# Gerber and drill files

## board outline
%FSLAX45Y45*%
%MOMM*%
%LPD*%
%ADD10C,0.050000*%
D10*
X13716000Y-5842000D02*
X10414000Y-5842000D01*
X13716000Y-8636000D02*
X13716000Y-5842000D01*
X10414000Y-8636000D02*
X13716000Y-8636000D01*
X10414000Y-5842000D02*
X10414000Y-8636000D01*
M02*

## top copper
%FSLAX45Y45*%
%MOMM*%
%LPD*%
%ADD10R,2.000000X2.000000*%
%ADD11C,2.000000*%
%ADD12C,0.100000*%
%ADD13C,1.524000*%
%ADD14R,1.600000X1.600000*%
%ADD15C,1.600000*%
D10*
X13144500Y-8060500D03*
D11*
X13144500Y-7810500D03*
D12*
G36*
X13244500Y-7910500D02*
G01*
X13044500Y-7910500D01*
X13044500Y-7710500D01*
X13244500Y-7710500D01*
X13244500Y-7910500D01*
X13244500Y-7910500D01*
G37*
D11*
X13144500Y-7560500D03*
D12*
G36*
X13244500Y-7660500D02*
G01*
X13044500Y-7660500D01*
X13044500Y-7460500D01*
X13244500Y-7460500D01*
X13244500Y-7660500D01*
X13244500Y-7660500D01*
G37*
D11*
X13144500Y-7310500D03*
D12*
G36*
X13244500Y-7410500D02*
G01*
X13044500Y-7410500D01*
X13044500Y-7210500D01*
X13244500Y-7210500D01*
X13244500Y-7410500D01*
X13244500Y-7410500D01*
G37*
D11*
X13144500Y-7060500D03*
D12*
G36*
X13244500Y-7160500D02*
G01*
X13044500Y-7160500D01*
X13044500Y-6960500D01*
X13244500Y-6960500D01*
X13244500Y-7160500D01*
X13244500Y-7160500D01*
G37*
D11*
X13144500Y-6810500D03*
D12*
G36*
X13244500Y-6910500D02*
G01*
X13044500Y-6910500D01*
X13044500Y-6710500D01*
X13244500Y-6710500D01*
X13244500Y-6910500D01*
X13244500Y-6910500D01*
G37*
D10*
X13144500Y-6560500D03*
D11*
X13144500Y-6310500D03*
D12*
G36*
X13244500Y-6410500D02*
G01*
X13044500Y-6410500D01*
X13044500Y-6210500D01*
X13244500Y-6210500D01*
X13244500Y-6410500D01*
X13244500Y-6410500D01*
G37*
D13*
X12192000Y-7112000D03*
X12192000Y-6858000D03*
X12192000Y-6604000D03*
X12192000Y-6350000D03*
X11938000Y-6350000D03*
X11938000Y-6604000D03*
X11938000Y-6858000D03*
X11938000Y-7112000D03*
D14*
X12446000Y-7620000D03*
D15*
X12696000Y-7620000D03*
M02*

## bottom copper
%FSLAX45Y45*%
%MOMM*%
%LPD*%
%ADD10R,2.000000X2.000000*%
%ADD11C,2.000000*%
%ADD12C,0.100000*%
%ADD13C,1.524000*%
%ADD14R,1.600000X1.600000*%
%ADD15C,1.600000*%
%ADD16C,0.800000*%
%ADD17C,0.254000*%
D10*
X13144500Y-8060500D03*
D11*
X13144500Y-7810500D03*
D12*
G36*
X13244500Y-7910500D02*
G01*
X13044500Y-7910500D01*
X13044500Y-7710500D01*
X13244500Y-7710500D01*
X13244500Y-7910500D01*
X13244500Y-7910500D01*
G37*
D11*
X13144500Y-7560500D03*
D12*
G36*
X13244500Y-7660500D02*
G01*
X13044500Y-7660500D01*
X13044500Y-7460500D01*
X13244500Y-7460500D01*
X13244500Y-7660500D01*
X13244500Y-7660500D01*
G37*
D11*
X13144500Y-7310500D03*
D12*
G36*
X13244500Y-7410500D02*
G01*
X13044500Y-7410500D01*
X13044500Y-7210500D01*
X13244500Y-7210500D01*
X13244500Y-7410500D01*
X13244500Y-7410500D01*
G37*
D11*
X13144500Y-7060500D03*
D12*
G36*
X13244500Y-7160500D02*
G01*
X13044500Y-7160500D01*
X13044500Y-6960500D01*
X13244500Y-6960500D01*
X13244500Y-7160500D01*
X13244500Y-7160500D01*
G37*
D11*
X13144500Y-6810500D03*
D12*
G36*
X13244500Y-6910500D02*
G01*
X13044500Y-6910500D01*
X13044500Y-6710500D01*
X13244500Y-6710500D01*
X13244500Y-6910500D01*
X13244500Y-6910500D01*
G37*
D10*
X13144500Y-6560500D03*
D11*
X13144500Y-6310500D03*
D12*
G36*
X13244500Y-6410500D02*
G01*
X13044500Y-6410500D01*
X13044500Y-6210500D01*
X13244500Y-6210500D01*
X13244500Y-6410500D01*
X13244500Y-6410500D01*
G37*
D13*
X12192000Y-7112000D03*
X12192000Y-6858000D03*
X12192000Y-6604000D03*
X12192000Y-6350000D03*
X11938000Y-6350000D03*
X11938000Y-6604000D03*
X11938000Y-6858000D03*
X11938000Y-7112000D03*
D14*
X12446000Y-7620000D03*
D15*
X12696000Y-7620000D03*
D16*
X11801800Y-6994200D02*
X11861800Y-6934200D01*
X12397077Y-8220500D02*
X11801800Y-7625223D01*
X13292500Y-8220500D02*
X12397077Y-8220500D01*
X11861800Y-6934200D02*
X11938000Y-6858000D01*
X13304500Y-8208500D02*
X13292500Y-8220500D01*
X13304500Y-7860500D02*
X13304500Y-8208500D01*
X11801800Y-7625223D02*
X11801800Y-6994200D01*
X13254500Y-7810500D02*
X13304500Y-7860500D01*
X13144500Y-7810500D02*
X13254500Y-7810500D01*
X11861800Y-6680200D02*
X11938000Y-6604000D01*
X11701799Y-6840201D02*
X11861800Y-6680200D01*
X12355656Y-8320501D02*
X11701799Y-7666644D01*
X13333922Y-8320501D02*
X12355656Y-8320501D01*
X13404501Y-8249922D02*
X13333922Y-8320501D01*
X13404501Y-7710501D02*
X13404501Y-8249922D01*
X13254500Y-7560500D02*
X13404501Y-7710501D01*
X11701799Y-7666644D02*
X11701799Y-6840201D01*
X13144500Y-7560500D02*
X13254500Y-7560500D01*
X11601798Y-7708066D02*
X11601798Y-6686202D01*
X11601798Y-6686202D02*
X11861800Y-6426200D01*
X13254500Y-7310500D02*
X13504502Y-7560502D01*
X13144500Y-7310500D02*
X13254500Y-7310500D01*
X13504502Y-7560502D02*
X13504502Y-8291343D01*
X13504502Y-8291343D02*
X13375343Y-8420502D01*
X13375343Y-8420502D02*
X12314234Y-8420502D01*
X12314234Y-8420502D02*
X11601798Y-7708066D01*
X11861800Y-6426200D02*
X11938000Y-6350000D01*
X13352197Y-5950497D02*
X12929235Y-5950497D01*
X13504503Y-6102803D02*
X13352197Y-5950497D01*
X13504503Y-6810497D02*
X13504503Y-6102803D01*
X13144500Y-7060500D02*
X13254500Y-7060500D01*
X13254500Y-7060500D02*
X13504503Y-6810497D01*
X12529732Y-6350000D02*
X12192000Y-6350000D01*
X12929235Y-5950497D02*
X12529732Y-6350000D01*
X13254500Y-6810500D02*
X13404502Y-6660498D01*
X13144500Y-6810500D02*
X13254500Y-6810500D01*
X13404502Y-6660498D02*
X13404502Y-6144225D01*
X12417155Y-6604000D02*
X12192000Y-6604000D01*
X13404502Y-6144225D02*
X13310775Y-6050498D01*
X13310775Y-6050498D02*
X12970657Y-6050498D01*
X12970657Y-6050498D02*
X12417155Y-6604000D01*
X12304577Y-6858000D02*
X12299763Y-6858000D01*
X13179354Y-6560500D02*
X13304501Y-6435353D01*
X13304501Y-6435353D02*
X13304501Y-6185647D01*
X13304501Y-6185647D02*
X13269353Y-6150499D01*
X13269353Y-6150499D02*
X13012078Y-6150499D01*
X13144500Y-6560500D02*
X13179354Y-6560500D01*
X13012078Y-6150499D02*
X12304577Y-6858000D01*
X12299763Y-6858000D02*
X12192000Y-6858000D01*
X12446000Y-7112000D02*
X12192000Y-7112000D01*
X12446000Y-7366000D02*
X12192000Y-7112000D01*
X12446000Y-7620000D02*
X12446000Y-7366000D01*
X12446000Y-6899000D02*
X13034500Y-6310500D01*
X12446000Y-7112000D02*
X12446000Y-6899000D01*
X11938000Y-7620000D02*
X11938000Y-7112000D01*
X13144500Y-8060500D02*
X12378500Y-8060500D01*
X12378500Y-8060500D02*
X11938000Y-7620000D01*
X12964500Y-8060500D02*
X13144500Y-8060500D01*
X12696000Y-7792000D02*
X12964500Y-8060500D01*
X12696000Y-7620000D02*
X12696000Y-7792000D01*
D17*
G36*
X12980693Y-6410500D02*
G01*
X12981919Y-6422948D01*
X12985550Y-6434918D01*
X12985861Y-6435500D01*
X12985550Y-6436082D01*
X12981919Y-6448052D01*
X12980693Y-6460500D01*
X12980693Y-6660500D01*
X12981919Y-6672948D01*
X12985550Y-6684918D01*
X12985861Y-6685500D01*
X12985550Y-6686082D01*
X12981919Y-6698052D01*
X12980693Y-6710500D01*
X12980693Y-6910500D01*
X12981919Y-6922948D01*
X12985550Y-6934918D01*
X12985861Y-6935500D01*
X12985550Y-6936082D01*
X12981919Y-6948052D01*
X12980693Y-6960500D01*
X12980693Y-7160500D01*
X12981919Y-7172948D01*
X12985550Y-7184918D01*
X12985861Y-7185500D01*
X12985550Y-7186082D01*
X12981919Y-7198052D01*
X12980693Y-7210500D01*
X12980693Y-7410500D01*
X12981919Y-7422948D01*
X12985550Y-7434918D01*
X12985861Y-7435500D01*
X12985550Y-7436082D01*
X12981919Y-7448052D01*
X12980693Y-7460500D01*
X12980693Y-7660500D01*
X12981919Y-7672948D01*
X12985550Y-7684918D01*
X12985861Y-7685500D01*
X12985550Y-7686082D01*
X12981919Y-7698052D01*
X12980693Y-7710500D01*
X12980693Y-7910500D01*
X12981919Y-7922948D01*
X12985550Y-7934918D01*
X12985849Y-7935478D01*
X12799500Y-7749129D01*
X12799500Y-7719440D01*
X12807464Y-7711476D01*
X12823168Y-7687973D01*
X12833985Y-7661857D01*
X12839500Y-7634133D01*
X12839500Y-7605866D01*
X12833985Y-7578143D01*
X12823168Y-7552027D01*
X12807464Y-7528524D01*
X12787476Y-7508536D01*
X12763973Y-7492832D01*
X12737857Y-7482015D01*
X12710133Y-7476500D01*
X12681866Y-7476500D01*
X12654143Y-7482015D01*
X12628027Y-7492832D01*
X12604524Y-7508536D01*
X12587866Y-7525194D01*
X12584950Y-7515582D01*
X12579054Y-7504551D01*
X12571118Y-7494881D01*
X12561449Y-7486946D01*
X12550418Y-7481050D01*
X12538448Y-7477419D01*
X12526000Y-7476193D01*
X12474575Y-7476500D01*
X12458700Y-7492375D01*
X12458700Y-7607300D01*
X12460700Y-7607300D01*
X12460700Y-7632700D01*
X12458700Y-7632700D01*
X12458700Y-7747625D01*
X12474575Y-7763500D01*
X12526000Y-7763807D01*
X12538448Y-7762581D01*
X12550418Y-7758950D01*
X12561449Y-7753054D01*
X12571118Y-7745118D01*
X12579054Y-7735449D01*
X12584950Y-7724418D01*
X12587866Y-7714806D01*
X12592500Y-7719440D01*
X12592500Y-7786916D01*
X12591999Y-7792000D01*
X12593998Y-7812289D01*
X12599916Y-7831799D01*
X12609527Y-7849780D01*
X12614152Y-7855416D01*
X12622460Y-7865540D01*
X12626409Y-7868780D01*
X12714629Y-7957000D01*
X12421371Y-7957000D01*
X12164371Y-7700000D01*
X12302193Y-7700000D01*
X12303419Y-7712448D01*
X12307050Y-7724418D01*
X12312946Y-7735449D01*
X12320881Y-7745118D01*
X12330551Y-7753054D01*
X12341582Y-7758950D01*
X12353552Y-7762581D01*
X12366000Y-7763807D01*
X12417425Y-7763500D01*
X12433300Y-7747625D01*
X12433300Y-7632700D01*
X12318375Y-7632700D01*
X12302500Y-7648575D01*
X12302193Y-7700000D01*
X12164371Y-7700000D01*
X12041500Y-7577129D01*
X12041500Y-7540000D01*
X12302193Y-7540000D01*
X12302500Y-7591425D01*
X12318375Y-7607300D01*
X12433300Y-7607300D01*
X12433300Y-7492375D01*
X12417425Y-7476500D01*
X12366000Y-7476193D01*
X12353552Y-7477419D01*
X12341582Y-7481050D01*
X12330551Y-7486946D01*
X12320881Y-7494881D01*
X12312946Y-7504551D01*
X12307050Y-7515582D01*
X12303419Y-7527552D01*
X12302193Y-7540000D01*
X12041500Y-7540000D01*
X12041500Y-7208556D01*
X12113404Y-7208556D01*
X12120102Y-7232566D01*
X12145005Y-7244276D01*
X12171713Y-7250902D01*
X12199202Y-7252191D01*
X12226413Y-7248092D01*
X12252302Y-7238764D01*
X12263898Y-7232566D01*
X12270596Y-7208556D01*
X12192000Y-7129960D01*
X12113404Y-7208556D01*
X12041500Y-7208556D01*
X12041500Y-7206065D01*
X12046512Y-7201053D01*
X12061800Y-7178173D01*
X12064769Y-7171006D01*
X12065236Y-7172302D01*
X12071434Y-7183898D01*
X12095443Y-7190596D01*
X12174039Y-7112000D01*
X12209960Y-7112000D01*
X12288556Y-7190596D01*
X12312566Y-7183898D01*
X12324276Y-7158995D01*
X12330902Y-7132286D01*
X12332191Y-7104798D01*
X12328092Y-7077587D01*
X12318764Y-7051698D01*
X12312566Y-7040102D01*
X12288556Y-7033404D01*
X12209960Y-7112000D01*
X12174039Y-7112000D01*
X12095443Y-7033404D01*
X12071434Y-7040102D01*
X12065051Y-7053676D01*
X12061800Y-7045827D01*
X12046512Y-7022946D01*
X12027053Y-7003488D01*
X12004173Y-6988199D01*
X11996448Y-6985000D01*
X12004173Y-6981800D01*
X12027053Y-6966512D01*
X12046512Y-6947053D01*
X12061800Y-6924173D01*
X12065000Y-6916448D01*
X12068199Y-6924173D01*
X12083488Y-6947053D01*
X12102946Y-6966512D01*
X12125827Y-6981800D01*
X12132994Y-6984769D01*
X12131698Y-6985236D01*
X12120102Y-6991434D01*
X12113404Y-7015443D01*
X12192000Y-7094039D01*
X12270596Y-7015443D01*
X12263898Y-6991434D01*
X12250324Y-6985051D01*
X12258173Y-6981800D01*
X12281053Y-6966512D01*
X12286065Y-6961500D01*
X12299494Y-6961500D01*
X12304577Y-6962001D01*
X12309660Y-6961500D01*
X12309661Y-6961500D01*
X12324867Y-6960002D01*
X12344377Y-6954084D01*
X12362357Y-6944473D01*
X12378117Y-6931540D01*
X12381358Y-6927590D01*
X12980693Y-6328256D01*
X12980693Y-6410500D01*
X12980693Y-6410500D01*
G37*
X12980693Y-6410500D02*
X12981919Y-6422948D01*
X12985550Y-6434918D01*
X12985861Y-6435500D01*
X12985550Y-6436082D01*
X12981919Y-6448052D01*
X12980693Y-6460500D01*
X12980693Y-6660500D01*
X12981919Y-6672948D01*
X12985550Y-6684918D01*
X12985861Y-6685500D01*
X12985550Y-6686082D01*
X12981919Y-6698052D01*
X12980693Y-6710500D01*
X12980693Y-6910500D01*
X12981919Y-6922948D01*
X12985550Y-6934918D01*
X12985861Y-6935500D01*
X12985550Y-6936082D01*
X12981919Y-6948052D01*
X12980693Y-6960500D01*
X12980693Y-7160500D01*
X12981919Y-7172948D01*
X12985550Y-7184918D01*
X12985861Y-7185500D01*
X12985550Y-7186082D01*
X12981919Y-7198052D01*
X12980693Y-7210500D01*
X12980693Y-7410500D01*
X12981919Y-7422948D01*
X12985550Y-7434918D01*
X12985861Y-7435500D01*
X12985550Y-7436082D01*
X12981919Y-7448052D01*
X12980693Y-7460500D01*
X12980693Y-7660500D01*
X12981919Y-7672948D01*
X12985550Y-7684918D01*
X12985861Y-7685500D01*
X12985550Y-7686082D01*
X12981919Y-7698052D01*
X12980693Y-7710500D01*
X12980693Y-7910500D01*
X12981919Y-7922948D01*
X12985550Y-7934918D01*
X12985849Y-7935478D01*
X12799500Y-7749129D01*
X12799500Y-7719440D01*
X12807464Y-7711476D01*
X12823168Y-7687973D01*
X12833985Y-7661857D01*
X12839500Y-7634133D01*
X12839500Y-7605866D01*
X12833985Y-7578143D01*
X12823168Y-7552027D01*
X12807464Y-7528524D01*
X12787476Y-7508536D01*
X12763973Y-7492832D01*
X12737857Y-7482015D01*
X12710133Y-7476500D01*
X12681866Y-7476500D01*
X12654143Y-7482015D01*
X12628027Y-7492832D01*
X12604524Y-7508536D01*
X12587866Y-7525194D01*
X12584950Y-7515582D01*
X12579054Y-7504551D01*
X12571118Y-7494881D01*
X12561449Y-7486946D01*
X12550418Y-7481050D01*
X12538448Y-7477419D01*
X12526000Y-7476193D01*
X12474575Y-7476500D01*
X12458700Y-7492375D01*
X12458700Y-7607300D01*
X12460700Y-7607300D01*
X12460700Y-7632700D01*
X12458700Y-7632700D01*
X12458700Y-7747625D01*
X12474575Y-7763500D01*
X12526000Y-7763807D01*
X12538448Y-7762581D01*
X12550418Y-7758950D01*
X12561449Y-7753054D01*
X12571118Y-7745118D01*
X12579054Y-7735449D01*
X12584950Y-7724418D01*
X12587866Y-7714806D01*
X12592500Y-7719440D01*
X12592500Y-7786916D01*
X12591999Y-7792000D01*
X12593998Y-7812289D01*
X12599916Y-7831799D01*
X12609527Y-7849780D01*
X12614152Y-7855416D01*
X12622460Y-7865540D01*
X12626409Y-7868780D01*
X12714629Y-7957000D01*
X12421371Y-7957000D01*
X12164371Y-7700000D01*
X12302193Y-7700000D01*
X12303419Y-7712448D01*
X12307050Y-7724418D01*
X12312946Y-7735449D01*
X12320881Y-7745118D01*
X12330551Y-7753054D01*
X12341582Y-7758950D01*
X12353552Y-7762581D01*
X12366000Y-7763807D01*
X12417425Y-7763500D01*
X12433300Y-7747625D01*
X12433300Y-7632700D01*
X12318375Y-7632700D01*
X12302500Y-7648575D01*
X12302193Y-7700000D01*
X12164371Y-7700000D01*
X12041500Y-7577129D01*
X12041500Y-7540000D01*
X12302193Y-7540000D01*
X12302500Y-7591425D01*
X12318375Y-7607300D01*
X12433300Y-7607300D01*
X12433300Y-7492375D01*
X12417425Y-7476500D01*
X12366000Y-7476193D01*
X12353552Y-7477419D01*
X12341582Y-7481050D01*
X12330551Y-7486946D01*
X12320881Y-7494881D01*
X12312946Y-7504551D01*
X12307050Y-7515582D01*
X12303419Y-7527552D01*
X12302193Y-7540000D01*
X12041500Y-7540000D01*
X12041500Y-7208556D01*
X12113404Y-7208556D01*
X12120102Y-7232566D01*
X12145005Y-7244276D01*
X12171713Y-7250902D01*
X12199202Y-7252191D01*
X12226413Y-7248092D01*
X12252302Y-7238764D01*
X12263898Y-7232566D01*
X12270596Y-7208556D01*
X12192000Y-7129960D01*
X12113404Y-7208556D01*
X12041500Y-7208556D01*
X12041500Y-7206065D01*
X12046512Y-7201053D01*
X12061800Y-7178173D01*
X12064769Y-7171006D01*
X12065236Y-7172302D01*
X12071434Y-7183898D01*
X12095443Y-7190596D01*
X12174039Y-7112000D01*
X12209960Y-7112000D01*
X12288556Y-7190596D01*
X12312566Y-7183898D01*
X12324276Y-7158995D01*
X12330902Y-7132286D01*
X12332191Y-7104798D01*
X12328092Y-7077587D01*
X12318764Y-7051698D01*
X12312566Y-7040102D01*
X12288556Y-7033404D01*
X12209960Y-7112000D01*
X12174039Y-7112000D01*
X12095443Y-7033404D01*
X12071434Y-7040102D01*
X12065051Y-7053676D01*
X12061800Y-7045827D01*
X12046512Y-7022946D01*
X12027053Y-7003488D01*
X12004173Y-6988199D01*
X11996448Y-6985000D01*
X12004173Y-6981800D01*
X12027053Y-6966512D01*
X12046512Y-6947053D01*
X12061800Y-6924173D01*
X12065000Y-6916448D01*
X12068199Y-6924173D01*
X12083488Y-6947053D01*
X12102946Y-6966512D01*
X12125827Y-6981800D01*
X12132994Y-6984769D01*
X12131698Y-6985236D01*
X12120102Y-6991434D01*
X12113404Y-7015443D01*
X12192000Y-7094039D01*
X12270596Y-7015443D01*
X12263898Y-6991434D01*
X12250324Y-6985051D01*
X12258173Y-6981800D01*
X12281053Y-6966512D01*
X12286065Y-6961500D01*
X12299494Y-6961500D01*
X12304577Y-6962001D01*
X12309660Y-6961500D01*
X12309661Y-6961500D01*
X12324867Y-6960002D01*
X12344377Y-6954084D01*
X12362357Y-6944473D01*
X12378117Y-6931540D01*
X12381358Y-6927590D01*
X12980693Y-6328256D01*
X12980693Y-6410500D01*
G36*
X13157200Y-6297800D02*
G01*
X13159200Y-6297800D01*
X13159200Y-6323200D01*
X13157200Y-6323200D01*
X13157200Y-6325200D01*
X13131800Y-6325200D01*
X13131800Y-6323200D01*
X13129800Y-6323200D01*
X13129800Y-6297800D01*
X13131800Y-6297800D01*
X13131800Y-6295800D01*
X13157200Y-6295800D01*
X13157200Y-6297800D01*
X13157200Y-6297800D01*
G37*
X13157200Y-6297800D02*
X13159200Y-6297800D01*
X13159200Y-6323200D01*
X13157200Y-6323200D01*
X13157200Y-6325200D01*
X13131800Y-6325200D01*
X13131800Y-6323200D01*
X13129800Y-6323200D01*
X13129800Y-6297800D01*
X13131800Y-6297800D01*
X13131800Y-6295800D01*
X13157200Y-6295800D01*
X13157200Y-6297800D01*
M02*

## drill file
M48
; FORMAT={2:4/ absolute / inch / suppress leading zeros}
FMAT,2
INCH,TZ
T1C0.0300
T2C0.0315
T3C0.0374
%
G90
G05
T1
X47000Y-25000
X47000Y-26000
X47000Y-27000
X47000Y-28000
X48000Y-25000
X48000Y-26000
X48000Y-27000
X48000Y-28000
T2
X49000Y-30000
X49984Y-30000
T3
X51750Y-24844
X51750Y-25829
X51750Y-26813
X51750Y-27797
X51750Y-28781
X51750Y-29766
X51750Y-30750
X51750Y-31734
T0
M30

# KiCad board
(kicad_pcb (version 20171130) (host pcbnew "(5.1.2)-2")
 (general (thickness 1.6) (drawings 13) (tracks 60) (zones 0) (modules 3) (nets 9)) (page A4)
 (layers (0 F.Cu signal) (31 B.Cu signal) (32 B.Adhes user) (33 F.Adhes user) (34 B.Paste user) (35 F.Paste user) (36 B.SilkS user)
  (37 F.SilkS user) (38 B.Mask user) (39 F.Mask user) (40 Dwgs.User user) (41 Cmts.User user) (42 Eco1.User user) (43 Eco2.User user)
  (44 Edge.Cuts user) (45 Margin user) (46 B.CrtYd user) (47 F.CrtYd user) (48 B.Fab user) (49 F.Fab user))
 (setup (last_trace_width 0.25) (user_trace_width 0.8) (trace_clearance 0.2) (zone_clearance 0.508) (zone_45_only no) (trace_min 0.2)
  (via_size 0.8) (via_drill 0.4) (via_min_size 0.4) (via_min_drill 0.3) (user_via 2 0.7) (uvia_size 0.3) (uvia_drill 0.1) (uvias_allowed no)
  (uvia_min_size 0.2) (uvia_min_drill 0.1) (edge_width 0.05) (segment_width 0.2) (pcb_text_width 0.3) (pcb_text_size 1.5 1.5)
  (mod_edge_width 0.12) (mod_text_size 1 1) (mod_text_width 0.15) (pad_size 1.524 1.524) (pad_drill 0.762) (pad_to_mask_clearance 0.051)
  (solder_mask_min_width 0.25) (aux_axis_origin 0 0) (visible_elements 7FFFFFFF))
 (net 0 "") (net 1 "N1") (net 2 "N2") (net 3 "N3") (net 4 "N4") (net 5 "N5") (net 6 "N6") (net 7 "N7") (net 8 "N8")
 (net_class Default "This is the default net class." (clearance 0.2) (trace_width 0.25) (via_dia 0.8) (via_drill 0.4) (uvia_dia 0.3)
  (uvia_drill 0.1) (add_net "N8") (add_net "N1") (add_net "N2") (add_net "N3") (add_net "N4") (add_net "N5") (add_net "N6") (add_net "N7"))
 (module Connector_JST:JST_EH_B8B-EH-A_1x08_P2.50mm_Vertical (layer F.Cu) (at 131.445 80.605 90)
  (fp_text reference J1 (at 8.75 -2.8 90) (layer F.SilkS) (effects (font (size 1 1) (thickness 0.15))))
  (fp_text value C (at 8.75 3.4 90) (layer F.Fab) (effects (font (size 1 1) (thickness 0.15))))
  (pad 1 thru_hole rect (at 0 0 90) (size 2 2) (drill 0.95) (layers *.Cu *.Mask) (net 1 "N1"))
  (pad 2 thru_hole trapezoid (at 2.5 0 90) (size 2 2) (drill 0.95) (layers *.Cu *.Mask) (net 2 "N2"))
  (pad 3 thru_hole trapezoid (at 5 0 90) (size 2 2) (drill 0.95) (layers *.Cu *.Mask) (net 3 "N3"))
  (pad 4 thru_hole trapezoid (at 7.5 0 90) (size 2 2) (drill 0.95) (layers *.Cu *.Mask) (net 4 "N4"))
  (pad 5 thru_hole trapezoid (at 10 0 90) (size 2 2) (drill 0.95) (layers *.Cu *.Mask) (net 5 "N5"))
  (pad 6 thru_hole trapezoid (at 12.5 0 90) (size 2 2) (drill 0.95) (layers *.Cu *.Mask) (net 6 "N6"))
  (pad 7 thru_hole rect (at 15 0 90) (size 2 2) (drill 0.95) (layers *.Cu *.Mask) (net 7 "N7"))
  (pad 8 thru_hole trapezoid (at 17.5 0 90) (size 2 2) (drill 0.95) (layers *.Cu *.Mask) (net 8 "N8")))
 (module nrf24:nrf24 (layer F.Cu) (at 114.3 63.5)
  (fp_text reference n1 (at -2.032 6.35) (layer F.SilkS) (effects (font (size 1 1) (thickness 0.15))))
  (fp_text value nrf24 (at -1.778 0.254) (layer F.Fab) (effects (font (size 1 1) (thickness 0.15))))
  (pad 0 thru_hole circle (at 7.62 7.62) (size 1.524 1.524) (drill 0.762) (layers *.Cu *.Mask) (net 8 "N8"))
  (pad 1 thru_hole circle (at 7.62 5.08) (size 1.524 1.524) (drill 0.762) (layers *.Cu *.Mask) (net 7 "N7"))
  (pad 2 thru_hole circle (at 7.62 2.54) (size 1.524 1.524) (drill 0.762) (layers *.Cu *.Mask) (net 6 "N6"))
  (pad 3 thru_hole circle (at 7.62 0) (size 1.524 1.524) (drill 0.762) (layers *.Cu *.Mask) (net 5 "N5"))
  (pad 4 thru_hole circle (at 5.08 0) (size 1.524 1.524) (drill 0.762) (layers *.Cu *.Mask) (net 4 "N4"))
  (pad 5 thru_hole circle (at 5.08 2.54) (size 1.524 1.524) (drill 0.762) (layers *.Cu *.Mask) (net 3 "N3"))
  (pad 6 thru_hole circle (at 5.08 5.08) (size 1.524 1.524) (drill 0.762) (layers *.Cu *.Mask) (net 2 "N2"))
  (pad 7 thru_hole circle (at 5.08 7.62) (size 1.524 1.524) (drill 0.762) (layers *.Cu *.Mask) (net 1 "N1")))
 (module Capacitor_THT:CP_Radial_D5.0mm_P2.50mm (layer F.Cu) (at 124.46 76.2)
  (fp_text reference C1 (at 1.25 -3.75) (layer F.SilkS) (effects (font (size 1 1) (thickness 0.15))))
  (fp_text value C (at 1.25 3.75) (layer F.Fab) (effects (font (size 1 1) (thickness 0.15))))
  (pad 1 thru_hole rect (at 0 0) (size 1.6 1.6) (drill 0.8) (layers *.Cu *.Mask) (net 8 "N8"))
  (pad 2 thru_hole circle (at 2.5 0) (size 1.6 1.6) (drill 0.8) (layers *.Cu *.Mask) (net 1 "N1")))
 (gr_line (start 137.16 58.42) (end 104.14 58.42) (layer Edge.Cuts) (width 0.05))
 (gr_line (start 137.16 86.36) (end 137.16 58.42) (layer Edge.Cuts) (width 0.05))
 (gr_line (start 104.14 86.36) (end 137.16 86.36) (layer Edge.Cuts) (width 0.05))
 (gr_line (start 104.14 58.42) (end 104.14 86.36) (layer Edge.Cuts) (width 0.05))
 (segment (start 118.017999 69.942001) (end 118.618001 69.341999) (width 0.8) (layer B.Cu) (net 2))
 (segment (start 123.970774 82.205001) (end 118.017999 76.252226) (width 0.8) (layer B.Cu) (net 2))
 (segment (start 132.925001 82.205001) (end 123.970774 82.205001) (width 0.8) (layer B.Cu) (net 2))
 (segment (start 118.618001 69.341999) (end 119.38 68.58) (width 0.8) (layer B.Cu) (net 2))
 (segment (start 133.045001 82.085001) (end 132.925001 82.205001) (width 0.8) (layer B.Cu) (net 2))
 (segment (start 133.045001 78.605001) (end 133.045001 82.085001) (width 0.8) (layer B.Cu) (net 2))
 (segment (start 118.017999 76.252226) (end 118.017999 69.942001) (width 0.8) (layer B.Cu) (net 2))
 (segment (start 132.545 78.105) (end 133.045001 78.605001) (width 0.8) (layer B.Cu) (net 2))
 (segment (start 131.445 78.105) (end 132.545 78.105) (width 0.8) (layer B.Cu) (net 2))
 (segment (start 118.618001 66.801999) (end 119.38 66.04) (width 0.8) (layer B.Cu) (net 3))
 (segment (start 117.017989 68.402011) (end 118.618001 66.801999) (width 0.8) (layer B.Cu) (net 3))
 (segment (start 123.556558 83.205011) (end 117.017989 76.666443) (width 0.8) (layer B.Cu) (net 3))
 (segment (start 133.339218 83.205011) (end 123.556558 83.205011) (width 0.8) (layer B.Cu) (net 3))
 (segment (start 134.045011 82.499218) (end 133.339218 83.205011) (width 0.8) (layer B.Cu) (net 3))
 (segment (start 134.045011 77.105011) (end 134.045011 82.499218) (width 0.8) (layer B.Cu) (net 3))
 (segment (start 132.545 75.605) (end 134.045011 77.105011) (width 0.8) (layer B.Cu) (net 3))
 (segment (start 117.017989 76.666443) (end 117.017989 68.402011) (width 0.8) (layer B.Cu) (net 3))
 (segment (start 131.445 75.605) (end 132.545 75.605) (width 0.8) (layer B.Cu) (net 3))
 (segment (start 116.017979 77.08066) (end 116.017979 66.862021) (width 0.8) (layer B.Cu) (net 4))
 (segment (start 116.017979 66.862021) (end 118.618001 64.261999) (width 0.8) (layer B.Cu) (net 4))
 (segment (start 132.545 73.105) (end 135.045021 75.605021) (width 0.8) (layer B.Cu) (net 4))
 (segment (start 131.445 73.105) (end 132.545 73.105) (width 0.8) (layer B.Cu) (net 4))
 (segment (start 135.045021 75.605021) (end 135.045021 82.913435) (width 0.8) (layer B.Cu) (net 4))
 (segment (start 135.045021 82.913435) (end 133.753435 84.205021) (width 0.8) (layer B.Cu) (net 4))
 (segment (start 133.753435 84.205021) (end 123.142341 84.205021) (width 0.8) (layer B.Cu) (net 4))
 (segment (start 123.142341 84.205021) (end 116.017979 77.08066) (width 0.8) (layer B.Cu) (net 4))
 (segment (start 118.618001 64.261999) (end 119.38 63.5) (width 0.8) (layer B.Cu) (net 4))
 (segment (start 133.521968 59.50497) (end 129.292351 59.50497) (width 0.8) (layer B.Cu) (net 5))
 (segment (start 135.04503 61.028032) (end 133.521968 59.50497) (width 0.8) (layer B.Cu) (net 5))
 (segment (start 135.04503 68.10497) (end 135.04503 61.028032) (width 0.8) (layer B.Cu) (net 5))
 (segment (start 131.445 70.605) (end 132.545 70.605) (width 0.8) (layer B.Cu) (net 5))
 (segment (start 132.545 70.605) (end 135.04503 68.10497) (width 0.8) (layer B.Cu) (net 5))
 (segment (start 125.297321 63.5) (end 121.92 63.5) (width 0.8) (layer B.Cu) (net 5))
 (segment (start 129.292351 59.50497) (end 125.297321 63.5) (width 0.8) (layer B.Cu) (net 5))
 (segment (start 132.545 68.105) (end 134.04502 66.60498) (width 0.8) (layer B.Cu) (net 6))
 (segment (start 131.445 68.105) (end 132.545 68.105) (width 0.8) (layer B.Cu) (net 6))
 (segment (start 134.04502 66.60498) (end 134.04502 61.442249) (width 0.8) (layer B.Cu) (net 6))
 (segment (start 124.171547 66.04) (end 121.92 66.04) (width 0.8) (layer B.Cu) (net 6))
 (segment (start 134.04502 61.442249) (end 133.107751 60.50498) (width 0.8) (layer B.Cu) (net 6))
 (segment (start 133.107751 60.50498) (end 129.706567 60.50498) (width 0.8) (layer B.Cu) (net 6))
 (segment (start 129.706567 60.50498) (end 124.171547 66.04) (width 0.8) (layer B.Cu) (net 6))
 (segment (start 123.045773 68.58) (end 122.99763 68.58) (width 0.8) (layer B.Cu) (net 7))
 (segment (start 131.793544 65.605) (end 133.04501 64.353534) (width 0.8) (layer B.Cu) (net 7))
 (segment (start 133.04501 64.353534) (end 133.04501 61.856466) (width 0.8) (layer B.Cu) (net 7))
 (segment (start 133.04501 61.856466) (end 132.693534 61.50499) (width 0.8) (layer B.Cu) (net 7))
 (segment (start 132.693534 61.50499) (end 130.120783 61.50499) (width 0.8) (layer B.Cu) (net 7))
 (segment (start 131.445 65.605) (end 131.793544 65.605) (width 0.8) (layer B.Cu) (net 7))
 (segment (start 130.120783 61.50499) (end 123.045773 68.58) (width 0.8) (layer B.Cu) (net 7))
 (segment (start 122.99763 68.58) (end 121.92 68.58) (width 0.8) (layer B.Cu) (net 7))
 (segment (start 124.46 71.12) (end 121.92 71.12) (width 0.8) (layer B.Cu) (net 8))
 (segment (start 124.46 73.66) (end 121.92 71.12) (width 0.8) (layer B.Cu) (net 8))
 (segment (start 124.46 76.2) (end 124.46 73.66) (width 0.8) (layer B.Cu) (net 8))
 (segment (start 124.46 68.99) (end 130.345 63.105) (width 0.8) (layer B.Cu) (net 8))
 (segment (start 124.46 71.12) (end 124.46 68.99) (width 0.8) (layer B.Cu) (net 8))
 (segment (start 119.38 76.2) (end 119.38 71.12) (width 0.8) (layer B.Cu) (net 1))
 (segment (start 131.445 80.605) (end 123.785 80.605) (width 0.8) (layer B.Cu) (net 1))
 (segment (start 123.785 80.605) (end 119.38 76.2) (width 0.8) (layer B.Cu) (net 1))
 (segment (start 129.645 80.605) (end 131.445 80.605) (width 0.8) (layer B.Cu) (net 1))
 (segment (start 126.96 77.92) (end 129.645 80.605) (width 0.8) (layer B.Cu) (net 1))
 (segment (start 126.96 76.2) (end 126.96 77.92) (width 0.8) (layer B.Cu) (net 1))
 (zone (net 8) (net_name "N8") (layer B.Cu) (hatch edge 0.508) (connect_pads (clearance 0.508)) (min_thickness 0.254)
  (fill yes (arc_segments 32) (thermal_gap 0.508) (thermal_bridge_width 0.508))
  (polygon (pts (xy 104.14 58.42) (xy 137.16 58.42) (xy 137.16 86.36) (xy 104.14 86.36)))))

